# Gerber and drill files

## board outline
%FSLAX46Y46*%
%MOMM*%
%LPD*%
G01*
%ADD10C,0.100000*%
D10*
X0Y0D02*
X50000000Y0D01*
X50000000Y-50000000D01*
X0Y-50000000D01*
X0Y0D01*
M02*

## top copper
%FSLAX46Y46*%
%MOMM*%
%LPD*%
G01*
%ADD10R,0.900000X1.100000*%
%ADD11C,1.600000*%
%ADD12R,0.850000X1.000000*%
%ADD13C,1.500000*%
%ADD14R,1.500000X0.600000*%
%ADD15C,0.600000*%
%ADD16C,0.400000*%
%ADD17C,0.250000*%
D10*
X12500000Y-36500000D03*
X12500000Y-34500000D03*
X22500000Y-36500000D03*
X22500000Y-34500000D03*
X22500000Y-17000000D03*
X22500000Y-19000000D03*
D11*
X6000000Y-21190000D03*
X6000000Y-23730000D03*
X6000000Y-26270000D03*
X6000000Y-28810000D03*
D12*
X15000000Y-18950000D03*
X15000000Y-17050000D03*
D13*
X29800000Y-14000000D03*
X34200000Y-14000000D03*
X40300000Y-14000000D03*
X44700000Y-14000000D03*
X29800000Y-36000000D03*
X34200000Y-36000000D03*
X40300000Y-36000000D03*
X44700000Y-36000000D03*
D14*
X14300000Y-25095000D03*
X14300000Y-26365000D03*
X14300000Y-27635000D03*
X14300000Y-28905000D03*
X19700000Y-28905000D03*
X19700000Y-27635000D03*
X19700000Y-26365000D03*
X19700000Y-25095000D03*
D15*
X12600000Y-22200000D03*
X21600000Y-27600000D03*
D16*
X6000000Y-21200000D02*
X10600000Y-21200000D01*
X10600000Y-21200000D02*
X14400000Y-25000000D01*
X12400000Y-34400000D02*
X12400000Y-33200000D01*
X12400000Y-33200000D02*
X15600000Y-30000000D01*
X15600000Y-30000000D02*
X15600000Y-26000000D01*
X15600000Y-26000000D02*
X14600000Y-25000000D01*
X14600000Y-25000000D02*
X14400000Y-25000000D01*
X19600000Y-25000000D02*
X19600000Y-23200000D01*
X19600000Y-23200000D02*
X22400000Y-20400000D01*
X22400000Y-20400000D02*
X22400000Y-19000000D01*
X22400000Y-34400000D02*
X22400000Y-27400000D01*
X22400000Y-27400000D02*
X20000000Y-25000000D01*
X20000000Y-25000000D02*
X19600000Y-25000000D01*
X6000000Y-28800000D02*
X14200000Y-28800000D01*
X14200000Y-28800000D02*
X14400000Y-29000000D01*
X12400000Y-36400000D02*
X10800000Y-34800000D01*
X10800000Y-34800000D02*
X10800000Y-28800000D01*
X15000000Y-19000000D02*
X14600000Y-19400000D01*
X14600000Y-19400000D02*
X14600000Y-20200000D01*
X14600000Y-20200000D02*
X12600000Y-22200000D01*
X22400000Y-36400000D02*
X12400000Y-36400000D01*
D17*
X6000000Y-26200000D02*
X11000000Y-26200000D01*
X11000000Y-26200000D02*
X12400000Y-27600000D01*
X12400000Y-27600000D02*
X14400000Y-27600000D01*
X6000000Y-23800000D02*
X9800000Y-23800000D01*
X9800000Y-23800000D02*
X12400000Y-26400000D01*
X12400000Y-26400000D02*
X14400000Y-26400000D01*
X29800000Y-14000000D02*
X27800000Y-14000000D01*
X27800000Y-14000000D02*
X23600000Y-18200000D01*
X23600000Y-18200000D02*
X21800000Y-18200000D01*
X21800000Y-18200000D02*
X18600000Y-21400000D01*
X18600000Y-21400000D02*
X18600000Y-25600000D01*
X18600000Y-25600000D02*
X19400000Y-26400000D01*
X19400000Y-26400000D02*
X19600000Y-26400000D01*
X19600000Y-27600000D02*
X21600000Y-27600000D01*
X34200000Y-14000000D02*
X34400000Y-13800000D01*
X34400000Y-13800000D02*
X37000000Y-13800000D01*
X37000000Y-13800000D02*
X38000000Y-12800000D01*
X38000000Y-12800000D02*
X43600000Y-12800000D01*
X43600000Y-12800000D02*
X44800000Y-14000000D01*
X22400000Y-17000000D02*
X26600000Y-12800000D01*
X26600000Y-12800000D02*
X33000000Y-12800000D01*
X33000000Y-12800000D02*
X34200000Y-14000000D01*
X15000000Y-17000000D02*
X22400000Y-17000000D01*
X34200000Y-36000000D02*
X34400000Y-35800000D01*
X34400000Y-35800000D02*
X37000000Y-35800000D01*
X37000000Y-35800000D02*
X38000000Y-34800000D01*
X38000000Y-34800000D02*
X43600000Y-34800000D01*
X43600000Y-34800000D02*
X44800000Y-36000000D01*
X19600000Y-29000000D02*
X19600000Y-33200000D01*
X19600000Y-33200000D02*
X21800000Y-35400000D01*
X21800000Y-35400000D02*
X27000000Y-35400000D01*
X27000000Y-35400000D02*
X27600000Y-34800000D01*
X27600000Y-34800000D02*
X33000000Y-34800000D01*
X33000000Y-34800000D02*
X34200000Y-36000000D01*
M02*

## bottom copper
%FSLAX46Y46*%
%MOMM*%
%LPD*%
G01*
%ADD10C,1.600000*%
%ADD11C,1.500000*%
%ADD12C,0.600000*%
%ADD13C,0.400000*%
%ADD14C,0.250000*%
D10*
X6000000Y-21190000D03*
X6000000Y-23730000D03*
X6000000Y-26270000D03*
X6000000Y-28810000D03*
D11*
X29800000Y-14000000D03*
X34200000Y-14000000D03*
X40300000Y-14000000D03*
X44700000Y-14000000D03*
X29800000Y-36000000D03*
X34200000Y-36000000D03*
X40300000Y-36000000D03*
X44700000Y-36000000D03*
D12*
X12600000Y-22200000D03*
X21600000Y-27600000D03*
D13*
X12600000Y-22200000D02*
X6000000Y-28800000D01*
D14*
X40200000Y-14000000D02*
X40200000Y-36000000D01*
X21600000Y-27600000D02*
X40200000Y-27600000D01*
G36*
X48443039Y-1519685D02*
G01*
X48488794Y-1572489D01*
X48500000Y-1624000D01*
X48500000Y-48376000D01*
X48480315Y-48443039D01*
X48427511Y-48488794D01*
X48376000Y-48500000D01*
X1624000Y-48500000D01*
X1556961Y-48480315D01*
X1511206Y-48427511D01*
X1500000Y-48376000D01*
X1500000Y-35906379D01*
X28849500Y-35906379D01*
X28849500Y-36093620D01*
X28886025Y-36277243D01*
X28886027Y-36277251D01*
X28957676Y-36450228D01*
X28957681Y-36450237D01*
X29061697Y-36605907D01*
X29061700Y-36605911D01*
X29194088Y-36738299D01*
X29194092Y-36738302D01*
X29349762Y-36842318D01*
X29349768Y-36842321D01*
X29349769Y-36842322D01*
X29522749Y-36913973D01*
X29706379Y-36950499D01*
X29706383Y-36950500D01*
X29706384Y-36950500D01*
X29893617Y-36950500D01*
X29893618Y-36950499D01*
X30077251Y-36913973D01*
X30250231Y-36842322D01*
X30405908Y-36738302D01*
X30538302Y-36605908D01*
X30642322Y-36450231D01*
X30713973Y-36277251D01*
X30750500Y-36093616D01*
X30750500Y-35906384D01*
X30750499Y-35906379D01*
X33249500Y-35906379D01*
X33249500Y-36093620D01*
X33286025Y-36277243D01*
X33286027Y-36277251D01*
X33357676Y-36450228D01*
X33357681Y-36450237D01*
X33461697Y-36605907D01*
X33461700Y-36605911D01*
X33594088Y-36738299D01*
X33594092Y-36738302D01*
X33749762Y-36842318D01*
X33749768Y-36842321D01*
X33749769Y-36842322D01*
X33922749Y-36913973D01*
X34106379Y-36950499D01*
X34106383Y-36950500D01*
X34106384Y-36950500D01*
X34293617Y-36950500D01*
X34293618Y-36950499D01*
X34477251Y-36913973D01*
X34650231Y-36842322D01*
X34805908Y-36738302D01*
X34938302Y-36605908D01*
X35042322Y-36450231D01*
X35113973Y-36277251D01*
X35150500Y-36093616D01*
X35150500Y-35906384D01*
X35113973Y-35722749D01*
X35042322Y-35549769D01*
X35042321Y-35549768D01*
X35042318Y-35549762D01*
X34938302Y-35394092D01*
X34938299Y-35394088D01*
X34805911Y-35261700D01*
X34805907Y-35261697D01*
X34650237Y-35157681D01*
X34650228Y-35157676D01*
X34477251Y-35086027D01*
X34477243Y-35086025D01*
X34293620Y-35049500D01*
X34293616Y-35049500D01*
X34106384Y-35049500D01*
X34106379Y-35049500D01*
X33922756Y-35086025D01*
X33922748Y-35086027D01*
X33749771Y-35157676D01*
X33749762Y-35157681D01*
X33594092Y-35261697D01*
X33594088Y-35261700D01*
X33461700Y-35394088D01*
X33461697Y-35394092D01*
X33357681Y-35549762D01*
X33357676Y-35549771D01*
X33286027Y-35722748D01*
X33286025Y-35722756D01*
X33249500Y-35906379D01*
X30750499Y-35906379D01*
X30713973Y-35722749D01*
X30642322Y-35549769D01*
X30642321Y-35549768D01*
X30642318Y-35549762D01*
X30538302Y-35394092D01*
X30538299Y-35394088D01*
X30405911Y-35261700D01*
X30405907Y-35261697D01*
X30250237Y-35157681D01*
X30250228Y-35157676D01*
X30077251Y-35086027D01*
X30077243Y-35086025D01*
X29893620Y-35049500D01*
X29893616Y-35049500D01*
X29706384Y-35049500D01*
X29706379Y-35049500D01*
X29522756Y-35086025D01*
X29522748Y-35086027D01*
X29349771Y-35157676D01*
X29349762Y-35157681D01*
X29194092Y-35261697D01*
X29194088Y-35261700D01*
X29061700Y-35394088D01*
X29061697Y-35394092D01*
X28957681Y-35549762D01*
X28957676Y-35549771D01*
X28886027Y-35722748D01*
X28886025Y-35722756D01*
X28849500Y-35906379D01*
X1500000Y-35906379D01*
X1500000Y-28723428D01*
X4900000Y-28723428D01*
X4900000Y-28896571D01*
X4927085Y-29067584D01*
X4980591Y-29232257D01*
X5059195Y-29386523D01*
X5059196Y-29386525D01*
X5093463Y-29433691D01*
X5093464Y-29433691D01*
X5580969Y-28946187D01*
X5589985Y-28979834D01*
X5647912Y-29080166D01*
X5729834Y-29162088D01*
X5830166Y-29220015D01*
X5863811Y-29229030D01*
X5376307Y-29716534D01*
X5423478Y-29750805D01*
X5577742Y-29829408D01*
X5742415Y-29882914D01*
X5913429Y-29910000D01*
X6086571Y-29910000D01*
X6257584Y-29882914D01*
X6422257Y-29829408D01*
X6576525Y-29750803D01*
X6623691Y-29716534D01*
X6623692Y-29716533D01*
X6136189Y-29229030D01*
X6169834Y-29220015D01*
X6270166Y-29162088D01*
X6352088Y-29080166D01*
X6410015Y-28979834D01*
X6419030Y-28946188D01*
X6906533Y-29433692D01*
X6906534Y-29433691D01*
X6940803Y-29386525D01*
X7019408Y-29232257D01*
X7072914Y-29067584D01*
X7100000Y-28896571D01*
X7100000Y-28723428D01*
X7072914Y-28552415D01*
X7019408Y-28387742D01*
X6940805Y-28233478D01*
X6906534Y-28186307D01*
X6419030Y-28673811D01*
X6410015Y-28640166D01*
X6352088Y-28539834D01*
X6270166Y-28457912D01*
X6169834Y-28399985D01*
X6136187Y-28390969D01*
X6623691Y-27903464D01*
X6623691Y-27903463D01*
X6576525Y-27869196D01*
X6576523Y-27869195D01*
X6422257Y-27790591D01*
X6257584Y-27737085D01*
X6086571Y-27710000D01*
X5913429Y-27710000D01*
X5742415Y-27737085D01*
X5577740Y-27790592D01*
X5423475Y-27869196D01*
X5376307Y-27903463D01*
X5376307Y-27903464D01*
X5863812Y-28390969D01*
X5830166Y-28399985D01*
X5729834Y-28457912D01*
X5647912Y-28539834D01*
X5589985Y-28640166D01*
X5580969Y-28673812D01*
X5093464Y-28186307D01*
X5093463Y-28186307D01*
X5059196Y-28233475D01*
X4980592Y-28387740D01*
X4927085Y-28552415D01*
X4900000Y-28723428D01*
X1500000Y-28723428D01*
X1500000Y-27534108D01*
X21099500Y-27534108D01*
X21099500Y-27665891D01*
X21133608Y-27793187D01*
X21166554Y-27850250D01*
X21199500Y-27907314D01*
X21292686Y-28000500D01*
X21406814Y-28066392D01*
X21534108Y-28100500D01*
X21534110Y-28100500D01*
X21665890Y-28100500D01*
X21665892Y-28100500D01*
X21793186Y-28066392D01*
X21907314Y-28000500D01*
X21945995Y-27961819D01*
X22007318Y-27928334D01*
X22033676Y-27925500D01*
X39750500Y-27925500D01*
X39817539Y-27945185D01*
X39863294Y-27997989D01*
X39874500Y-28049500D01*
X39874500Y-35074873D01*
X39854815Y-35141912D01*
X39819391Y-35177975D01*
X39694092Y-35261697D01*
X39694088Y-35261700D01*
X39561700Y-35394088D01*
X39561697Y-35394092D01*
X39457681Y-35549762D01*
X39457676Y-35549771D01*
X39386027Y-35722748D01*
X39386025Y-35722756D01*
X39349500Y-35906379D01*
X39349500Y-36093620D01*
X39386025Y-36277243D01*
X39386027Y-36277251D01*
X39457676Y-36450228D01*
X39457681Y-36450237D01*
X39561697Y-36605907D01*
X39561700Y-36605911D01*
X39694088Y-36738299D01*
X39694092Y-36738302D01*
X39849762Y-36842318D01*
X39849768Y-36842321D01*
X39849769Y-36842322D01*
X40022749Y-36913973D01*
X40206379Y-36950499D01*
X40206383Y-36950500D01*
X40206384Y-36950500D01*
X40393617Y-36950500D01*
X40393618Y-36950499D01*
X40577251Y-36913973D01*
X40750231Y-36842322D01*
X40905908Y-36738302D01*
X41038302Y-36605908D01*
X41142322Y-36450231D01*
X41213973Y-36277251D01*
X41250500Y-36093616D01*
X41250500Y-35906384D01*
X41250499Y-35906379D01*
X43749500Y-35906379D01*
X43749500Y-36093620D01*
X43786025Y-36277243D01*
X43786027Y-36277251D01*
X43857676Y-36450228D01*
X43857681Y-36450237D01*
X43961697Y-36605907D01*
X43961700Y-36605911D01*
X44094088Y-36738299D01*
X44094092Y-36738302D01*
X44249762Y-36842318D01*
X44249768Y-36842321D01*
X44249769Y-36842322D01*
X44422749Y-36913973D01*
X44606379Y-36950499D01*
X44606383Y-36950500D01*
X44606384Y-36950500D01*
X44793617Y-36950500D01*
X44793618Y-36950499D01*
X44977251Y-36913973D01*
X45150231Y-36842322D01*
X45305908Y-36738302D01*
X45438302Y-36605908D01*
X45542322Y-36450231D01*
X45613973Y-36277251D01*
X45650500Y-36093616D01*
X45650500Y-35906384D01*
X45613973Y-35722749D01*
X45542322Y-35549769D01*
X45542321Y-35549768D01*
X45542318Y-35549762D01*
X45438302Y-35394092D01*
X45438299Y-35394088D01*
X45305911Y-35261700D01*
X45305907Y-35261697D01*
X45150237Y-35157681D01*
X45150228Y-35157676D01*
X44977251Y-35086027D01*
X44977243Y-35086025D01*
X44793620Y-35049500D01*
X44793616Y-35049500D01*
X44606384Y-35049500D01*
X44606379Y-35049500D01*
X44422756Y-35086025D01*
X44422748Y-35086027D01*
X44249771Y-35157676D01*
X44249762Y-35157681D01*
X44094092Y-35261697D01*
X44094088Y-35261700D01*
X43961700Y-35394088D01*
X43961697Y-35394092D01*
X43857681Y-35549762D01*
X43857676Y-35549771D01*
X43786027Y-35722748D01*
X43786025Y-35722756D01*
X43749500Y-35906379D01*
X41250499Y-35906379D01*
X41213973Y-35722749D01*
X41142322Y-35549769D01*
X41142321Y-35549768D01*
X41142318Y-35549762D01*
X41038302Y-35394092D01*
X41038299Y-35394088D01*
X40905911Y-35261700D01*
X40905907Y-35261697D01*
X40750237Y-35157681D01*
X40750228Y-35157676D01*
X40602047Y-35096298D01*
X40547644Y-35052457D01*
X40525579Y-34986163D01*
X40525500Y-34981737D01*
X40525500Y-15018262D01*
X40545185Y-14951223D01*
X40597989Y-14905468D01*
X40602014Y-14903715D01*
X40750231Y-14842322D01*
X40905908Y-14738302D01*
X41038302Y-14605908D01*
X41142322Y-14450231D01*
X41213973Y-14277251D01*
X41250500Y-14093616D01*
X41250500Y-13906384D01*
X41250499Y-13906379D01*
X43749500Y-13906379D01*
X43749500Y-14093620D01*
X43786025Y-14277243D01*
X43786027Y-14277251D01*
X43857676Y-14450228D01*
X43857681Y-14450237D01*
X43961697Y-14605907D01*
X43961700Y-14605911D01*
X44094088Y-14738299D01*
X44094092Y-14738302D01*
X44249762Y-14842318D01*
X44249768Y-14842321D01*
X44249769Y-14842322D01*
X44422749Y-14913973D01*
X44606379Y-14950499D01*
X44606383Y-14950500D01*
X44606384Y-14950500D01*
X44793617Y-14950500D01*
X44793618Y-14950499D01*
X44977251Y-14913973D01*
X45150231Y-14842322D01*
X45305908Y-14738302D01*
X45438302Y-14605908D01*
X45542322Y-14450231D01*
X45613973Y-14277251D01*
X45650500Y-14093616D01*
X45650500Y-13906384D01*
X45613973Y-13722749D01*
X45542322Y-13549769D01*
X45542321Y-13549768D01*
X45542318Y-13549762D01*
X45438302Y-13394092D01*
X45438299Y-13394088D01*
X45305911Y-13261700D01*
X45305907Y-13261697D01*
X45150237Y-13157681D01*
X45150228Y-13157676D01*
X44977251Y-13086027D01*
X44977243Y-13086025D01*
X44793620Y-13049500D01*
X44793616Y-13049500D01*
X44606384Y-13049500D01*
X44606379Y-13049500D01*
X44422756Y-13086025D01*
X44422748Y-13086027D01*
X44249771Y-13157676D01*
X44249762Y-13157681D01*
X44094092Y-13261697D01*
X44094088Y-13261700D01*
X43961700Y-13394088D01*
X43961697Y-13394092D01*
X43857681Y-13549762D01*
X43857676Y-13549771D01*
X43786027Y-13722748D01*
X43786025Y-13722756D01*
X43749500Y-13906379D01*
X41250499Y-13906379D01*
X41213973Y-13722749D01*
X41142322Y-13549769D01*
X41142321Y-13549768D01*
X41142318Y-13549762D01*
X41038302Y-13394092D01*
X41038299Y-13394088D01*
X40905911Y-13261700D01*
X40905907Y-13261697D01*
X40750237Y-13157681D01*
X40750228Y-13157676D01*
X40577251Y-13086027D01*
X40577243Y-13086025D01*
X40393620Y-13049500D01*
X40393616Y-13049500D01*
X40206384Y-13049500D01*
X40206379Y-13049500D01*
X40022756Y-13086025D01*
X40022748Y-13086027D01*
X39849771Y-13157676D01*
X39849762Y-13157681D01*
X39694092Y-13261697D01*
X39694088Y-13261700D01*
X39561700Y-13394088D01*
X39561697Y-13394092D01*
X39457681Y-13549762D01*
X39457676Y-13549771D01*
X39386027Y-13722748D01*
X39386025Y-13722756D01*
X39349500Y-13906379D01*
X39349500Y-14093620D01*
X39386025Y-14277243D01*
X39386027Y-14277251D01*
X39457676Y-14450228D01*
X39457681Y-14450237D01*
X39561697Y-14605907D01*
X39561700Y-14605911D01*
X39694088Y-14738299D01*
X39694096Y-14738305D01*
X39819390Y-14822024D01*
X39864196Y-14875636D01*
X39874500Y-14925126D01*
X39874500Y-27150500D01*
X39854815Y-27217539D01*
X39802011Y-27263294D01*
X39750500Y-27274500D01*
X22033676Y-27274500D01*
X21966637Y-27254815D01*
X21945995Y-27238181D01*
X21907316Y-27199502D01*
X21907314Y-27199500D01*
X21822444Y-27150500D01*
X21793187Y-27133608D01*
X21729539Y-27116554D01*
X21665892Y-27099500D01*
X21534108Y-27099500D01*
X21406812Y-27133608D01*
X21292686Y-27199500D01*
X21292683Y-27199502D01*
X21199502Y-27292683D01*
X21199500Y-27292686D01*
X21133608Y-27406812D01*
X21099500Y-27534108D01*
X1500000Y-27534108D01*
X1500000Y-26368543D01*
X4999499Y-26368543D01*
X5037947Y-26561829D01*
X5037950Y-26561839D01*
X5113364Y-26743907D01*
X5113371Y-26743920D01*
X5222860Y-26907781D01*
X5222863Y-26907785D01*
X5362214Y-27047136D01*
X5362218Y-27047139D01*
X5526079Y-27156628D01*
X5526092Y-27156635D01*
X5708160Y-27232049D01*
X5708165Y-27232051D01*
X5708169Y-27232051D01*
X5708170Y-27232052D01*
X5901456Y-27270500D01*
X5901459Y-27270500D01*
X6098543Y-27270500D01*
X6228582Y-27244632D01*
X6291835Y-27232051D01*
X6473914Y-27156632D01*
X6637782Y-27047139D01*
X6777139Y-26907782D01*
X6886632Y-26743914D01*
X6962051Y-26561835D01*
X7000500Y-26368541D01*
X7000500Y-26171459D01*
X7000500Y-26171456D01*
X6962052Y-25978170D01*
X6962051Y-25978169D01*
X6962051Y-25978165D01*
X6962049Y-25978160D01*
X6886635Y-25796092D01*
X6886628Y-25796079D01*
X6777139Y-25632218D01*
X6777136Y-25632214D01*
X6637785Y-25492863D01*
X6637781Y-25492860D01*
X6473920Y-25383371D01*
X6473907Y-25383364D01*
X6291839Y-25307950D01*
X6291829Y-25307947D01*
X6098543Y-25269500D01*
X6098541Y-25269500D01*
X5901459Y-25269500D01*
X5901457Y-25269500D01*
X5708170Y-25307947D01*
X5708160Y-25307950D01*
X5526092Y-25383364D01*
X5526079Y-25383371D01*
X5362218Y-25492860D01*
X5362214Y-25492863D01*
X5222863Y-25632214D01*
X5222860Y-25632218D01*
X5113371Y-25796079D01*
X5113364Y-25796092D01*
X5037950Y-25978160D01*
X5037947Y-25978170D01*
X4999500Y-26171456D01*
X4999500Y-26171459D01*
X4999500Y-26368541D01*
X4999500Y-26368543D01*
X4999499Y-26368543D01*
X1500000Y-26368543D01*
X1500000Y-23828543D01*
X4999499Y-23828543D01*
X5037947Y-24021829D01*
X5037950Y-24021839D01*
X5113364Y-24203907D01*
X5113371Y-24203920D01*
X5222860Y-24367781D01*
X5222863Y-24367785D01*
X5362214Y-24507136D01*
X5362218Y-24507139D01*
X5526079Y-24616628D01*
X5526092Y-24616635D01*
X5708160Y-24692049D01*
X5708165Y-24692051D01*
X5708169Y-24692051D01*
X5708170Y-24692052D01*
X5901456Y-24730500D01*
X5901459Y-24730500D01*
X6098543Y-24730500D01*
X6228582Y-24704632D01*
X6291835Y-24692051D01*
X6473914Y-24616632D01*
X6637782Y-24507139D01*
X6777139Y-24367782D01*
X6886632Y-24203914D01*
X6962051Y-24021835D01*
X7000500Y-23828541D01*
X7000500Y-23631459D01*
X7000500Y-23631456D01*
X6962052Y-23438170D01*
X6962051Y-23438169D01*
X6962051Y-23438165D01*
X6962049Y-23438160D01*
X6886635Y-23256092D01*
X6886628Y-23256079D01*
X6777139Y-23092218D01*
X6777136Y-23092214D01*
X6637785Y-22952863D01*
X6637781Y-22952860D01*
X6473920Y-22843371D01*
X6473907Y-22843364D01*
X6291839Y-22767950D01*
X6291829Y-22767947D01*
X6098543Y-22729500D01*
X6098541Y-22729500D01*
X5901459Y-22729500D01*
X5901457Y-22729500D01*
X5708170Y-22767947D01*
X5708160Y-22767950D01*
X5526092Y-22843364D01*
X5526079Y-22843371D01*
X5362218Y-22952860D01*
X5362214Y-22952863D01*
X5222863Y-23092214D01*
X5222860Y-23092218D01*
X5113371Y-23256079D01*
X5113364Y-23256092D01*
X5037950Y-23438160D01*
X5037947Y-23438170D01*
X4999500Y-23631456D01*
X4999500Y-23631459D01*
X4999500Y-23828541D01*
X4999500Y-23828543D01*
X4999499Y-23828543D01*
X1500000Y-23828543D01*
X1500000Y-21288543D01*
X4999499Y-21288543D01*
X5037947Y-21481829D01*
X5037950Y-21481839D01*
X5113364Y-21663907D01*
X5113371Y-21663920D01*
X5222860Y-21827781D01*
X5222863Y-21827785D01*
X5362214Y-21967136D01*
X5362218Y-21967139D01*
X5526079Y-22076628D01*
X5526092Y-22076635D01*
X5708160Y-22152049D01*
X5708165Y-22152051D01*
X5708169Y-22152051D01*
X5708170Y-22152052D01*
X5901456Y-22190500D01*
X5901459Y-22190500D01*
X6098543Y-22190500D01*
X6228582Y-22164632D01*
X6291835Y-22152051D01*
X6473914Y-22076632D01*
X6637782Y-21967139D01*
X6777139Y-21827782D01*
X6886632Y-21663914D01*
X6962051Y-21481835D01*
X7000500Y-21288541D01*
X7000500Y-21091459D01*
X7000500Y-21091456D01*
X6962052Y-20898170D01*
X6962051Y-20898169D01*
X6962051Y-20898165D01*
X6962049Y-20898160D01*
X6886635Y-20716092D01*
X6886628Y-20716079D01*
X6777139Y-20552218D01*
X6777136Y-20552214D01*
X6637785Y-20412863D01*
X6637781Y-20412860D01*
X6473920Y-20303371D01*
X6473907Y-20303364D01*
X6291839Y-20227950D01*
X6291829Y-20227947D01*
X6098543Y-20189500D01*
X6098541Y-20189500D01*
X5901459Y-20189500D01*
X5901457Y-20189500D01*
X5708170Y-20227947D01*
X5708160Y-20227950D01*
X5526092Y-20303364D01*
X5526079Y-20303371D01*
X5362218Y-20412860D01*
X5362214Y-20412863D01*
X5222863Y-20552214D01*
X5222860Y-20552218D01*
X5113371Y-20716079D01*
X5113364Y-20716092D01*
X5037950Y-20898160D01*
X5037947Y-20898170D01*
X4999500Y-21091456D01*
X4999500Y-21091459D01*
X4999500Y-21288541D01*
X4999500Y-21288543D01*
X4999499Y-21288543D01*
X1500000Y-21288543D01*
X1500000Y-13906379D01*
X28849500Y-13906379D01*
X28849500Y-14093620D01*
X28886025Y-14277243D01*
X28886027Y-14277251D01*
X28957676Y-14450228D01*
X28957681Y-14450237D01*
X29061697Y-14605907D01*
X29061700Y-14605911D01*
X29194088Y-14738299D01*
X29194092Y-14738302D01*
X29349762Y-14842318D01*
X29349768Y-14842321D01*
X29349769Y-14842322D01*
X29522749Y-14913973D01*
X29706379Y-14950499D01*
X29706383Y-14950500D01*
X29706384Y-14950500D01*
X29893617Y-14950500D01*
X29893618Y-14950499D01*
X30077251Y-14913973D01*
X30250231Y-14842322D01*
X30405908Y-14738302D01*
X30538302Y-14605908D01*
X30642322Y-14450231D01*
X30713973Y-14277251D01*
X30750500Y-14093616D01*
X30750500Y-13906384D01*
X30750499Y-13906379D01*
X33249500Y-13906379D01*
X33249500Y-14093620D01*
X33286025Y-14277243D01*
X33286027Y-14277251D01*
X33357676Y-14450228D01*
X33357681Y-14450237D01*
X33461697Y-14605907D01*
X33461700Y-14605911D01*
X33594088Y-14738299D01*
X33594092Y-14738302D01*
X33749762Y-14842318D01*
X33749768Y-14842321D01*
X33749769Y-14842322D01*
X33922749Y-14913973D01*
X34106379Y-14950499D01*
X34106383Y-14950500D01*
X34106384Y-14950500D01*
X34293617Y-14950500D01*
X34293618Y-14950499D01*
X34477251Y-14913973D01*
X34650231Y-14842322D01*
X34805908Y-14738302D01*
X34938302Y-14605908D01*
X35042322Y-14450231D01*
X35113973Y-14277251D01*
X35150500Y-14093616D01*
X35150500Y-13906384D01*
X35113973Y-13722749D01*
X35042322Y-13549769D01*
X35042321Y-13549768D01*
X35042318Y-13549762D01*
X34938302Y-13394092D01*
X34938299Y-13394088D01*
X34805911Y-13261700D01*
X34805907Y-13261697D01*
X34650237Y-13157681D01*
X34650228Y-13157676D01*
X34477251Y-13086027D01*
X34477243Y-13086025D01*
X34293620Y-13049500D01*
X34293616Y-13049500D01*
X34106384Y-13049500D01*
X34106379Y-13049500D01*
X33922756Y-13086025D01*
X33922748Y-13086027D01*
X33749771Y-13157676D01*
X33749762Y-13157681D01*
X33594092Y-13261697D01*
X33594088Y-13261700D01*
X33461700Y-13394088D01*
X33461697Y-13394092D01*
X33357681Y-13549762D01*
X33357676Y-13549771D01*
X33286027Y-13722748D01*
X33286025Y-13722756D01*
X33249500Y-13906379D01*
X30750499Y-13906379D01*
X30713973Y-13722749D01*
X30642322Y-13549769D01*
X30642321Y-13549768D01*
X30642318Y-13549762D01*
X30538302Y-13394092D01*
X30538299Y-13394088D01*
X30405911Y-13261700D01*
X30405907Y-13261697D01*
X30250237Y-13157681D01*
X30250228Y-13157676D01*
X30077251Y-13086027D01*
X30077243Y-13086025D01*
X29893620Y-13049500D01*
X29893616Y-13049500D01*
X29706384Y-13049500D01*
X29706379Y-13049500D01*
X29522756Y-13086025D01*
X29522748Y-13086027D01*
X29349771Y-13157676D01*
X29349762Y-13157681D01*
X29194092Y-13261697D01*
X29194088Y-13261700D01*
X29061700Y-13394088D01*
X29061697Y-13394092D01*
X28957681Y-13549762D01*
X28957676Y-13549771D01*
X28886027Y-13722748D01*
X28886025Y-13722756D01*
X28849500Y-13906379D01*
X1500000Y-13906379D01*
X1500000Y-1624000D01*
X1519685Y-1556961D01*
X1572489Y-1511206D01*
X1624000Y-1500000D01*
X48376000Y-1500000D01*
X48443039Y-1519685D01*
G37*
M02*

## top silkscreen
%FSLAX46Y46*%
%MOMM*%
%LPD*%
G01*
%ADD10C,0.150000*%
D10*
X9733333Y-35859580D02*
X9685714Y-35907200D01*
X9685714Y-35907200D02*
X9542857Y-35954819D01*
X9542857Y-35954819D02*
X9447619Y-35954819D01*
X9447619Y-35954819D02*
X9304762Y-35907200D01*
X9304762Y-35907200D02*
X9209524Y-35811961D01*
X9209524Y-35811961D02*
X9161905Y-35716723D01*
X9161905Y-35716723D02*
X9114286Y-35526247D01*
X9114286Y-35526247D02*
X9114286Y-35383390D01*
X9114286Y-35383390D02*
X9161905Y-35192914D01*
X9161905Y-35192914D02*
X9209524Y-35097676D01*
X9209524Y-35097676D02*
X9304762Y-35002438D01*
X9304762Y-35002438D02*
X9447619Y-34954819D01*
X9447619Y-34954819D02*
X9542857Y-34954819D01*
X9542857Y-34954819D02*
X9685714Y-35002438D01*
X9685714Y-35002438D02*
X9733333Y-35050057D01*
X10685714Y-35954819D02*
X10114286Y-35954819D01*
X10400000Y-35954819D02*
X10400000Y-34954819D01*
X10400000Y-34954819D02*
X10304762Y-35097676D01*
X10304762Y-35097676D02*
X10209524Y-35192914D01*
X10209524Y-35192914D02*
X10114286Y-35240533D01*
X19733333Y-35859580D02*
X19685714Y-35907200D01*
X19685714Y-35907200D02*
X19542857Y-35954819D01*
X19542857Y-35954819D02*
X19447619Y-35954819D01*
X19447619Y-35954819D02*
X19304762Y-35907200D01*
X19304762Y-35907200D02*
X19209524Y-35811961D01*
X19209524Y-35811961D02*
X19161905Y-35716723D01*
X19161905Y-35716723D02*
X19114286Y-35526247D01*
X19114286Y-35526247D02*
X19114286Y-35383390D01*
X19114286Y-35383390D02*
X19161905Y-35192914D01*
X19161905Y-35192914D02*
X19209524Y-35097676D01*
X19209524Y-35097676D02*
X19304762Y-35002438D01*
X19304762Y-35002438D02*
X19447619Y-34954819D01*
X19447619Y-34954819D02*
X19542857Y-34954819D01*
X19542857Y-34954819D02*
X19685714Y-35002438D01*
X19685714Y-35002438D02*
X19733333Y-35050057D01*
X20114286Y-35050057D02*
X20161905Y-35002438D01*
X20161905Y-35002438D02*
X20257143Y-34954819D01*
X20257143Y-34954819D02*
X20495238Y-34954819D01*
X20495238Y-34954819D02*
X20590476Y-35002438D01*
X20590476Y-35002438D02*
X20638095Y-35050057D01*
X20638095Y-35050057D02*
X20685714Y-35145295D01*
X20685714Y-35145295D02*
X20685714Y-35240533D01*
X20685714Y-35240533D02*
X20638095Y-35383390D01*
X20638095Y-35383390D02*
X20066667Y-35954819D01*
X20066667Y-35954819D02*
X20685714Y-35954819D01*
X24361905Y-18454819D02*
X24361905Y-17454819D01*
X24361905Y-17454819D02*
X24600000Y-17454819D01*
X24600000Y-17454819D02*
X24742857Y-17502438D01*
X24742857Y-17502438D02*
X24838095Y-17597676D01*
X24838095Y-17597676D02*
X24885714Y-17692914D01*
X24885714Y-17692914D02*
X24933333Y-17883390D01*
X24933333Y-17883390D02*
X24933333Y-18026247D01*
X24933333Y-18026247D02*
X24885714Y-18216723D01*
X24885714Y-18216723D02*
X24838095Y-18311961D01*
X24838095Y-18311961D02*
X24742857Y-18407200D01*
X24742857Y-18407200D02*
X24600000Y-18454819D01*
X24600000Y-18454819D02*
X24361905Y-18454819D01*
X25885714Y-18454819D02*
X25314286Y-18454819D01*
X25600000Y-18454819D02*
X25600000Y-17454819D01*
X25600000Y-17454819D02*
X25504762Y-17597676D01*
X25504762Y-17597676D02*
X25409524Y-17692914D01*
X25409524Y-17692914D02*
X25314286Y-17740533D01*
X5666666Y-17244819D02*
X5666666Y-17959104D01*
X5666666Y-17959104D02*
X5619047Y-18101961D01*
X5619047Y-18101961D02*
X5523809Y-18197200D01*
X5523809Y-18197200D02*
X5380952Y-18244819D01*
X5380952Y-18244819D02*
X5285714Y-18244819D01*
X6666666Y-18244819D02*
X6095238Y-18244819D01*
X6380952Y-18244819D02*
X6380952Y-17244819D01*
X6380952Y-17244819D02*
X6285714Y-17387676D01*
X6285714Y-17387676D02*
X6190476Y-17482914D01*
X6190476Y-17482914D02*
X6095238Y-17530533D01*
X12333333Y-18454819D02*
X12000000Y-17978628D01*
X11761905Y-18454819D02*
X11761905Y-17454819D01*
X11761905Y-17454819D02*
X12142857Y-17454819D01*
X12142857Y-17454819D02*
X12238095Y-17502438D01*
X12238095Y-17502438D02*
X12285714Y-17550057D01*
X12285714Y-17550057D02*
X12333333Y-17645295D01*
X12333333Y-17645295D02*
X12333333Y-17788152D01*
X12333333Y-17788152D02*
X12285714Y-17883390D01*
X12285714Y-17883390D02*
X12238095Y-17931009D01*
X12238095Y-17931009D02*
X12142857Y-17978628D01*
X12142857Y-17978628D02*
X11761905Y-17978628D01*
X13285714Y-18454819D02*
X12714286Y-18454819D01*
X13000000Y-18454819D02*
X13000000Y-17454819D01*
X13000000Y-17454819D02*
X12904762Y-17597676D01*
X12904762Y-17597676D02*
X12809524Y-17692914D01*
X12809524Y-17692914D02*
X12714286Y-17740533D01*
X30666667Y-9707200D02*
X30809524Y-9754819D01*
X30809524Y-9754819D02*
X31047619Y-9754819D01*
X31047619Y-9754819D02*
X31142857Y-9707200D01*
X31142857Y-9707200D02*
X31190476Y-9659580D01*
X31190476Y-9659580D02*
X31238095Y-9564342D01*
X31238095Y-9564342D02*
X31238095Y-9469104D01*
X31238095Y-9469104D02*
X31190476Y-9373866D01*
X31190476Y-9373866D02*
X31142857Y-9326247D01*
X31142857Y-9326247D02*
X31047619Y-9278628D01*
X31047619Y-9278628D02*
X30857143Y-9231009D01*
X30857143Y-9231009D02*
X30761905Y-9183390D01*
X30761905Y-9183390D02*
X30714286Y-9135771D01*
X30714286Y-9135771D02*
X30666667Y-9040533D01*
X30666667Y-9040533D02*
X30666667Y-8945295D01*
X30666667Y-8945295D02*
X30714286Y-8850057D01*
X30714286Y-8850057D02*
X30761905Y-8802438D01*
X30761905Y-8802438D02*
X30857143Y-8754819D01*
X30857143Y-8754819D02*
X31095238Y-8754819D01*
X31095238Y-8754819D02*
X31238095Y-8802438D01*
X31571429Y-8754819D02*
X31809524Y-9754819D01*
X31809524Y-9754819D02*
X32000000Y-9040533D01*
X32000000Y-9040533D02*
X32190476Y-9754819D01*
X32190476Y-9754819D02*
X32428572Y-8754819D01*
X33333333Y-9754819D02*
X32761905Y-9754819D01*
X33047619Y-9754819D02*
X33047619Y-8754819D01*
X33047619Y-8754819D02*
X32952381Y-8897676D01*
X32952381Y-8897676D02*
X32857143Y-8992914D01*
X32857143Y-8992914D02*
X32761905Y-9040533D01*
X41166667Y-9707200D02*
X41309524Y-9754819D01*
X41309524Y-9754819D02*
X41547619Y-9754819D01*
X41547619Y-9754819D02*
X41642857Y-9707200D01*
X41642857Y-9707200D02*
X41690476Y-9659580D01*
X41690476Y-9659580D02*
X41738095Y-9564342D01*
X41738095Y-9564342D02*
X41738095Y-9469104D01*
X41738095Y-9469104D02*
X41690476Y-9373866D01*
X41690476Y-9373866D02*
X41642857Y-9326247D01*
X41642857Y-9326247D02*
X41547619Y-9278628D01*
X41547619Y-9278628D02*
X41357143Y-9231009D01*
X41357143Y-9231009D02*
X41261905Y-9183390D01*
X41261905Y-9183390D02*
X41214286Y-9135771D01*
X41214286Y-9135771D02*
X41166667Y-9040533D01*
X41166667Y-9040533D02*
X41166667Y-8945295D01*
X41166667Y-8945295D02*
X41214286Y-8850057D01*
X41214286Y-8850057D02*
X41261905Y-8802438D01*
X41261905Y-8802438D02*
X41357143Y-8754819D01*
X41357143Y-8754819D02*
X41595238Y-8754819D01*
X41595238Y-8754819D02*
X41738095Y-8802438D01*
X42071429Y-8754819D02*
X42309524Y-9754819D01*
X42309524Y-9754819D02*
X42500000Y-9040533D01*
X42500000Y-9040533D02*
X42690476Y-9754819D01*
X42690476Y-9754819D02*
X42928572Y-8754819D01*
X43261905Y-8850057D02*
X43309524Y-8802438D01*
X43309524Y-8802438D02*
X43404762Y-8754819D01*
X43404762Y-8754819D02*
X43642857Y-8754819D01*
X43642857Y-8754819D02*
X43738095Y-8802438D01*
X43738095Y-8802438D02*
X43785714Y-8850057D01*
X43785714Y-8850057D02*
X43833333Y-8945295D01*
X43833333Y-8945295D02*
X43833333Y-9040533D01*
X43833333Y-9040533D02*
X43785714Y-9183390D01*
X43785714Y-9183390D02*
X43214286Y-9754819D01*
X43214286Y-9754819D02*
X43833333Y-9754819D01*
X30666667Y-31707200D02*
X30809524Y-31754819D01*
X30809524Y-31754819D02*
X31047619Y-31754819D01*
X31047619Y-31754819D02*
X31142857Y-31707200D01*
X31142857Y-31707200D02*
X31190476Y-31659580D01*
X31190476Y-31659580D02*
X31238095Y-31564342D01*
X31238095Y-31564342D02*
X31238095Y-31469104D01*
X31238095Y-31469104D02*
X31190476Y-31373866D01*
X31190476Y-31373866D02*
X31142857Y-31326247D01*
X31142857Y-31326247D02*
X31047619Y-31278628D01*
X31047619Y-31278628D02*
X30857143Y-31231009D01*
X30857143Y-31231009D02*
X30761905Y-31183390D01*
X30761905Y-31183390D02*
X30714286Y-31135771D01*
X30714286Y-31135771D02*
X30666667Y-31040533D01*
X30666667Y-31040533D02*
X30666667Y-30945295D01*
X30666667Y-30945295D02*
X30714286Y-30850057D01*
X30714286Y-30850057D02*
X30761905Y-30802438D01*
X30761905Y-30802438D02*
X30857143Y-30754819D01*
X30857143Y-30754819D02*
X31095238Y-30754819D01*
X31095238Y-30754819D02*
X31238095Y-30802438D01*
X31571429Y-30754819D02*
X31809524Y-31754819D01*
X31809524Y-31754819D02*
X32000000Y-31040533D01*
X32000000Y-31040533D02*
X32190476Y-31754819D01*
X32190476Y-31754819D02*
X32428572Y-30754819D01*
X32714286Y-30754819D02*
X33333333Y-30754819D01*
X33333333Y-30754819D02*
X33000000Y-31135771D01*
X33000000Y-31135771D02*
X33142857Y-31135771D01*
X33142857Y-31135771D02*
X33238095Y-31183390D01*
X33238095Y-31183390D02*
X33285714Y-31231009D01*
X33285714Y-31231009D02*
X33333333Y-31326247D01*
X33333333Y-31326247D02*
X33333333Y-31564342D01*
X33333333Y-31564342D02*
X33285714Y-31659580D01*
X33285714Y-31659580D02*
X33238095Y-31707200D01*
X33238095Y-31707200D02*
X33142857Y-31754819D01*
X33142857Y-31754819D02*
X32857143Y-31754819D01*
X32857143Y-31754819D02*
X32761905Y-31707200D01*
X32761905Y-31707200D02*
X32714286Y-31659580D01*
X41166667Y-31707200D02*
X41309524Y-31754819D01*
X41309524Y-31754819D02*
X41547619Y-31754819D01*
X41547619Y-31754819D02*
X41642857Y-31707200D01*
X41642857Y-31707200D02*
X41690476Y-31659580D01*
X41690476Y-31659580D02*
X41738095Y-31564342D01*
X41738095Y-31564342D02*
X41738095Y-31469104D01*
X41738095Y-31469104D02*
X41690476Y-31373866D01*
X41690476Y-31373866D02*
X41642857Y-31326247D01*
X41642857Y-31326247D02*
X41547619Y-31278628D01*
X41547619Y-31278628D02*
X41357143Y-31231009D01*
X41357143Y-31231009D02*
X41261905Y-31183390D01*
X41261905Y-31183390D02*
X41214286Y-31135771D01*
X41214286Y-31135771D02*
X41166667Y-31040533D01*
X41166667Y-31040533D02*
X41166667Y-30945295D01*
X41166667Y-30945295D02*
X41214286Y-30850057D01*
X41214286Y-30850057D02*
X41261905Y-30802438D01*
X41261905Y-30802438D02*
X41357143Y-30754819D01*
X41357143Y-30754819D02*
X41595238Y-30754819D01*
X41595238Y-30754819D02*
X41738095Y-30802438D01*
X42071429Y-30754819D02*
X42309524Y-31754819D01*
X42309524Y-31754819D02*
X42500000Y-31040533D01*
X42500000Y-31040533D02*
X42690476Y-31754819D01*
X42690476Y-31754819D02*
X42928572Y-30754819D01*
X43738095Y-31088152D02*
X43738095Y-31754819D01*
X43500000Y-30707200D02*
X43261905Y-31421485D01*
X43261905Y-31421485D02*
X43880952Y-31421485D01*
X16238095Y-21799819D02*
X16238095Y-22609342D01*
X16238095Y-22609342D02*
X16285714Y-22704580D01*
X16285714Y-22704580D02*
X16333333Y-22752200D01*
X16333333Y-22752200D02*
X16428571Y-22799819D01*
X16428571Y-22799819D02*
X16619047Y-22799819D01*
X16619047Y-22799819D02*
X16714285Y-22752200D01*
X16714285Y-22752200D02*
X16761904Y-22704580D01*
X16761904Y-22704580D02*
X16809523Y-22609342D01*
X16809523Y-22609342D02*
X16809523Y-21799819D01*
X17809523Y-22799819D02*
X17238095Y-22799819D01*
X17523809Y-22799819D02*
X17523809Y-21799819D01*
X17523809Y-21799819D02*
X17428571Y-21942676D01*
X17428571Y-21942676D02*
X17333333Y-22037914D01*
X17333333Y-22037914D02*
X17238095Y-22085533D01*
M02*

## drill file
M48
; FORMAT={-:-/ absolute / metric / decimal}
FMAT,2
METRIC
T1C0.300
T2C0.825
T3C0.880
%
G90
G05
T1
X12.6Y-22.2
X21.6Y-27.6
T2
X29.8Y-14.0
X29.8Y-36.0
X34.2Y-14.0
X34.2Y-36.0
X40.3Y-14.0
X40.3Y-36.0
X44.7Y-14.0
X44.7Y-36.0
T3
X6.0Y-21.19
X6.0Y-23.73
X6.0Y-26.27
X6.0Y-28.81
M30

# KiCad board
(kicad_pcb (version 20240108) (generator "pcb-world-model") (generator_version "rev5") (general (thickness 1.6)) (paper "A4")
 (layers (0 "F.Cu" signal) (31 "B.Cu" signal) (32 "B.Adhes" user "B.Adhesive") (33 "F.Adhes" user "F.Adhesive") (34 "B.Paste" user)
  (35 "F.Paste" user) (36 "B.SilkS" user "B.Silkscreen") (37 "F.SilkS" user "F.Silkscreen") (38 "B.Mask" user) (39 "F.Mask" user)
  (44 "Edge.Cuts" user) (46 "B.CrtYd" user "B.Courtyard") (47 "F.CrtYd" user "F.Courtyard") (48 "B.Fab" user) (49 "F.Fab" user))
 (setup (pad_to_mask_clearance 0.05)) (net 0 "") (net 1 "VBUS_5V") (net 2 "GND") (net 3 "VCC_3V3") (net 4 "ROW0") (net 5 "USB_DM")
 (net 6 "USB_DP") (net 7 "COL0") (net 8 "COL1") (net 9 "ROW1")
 (gr_rect (start 0.0 0.0) (end 50.0000 50.0000) (stroke (width 0.1) (type default)) (fill none) (layer "Edge.Cuts"))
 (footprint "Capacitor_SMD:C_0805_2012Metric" (layer "F.Cu") (at 12.5000 35.5000 90)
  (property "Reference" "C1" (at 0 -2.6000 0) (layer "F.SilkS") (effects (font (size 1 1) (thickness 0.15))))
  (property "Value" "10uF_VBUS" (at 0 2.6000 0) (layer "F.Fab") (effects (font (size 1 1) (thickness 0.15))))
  (pad "1" smd rect (at -1.0000 0.0000) (size 0.9000 1.1000) (layers "F.Cu" "F.Paste" "F.Mask") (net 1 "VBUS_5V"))
  (pad "2" smd rect (at 1.0000 0.0000) (size 0.9000 1.1000) (layers "F.Cu" "F.Paste" "F.Mask") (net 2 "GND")))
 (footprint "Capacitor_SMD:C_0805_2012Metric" (layer "F.Cu") (at 22.5000 35.5000 90)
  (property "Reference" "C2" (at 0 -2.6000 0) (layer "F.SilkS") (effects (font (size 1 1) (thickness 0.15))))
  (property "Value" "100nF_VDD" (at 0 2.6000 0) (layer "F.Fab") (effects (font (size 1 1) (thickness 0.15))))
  (pad "1" smd rect (at -1.0000 0.0000) (size 0.9000 1.1000) (layers "F.Cu" "F.Paste" "F.Mask") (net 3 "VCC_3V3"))
  (pad "2" smd rect (at 1.0000 0.0000) (size 0.9000 1.1000) (layers "F.Cu" "F.Paste" "F.Mask") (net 2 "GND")))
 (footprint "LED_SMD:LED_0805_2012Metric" (layer "F.Cu") (at 22.5000 18.0000 270)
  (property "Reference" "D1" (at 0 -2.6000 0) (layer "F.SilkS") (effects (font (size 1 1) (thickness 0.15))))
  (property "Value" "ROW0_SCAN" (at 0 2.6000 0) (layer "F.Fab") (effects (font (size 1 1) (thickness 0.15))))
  (pad "1" smd rect (at -1.0000 0.0000) (size 0.9000 1.1000) (layers "F.Cu" "F.Paste" "F.Mask") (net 3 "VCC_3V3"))
  (pad "2" smd rect (at 1.0000 0.0000) (size 0.9000 1.1000) (layers "F.Cu" "F.Paste" "F.Mask") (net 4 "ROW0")))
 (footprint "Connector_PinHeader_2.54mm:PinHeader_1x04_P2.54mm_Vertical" (layer "F.Cu") (at 6.0000 25.0000 0) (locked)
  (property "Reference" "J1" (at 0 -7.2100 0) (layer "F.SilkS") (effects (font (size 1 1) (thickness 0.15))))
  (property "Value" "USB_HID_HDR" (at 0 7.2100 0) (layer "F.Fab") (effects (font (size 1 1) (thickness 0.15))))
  (pad "1" thru_hole circle (at 0.0000 -3.8100) (size 1.6000 1.6000) (drill 0.8800) (layers "*.Cu" "*.Mask") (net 1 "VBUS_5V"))
  (pad "2" thru_hole circle (at 0.0000 -1.2700) (size 1.6000 1.6000) (drill 0.8800) (layers "*.Cu" "*.Mask") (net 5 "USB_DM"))
  (pad "3" thru_hole circle (at 0.0000 1.2700) (size 1.6000 1.6000) (drill 0.8800) (layers "*.Cu" "*.Mask") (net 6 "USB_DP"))
  (pad "4" thru_hole circle (at 0.0000 3.8100) (size 1.6000 1.6000) (drill 0.8800) (layers "*.Cu" "*.Mask") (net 2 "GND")))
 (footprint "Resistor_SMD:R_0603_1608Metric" (layer "F.Cu") (at 15.0000 18.0000 90)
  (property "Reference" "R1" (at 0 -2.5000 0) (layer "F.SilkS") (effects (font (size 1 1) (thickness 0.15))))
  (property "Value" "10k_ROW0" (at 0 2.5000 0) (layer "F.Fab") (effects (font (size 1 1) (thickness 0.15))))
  (pad "1" smd rect (at -0.9500 0.0000) (size 0.8500 1.0000) (layers "F.Cu" "F.Paste" "F.Mask") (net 4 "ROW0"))
  (pad "2" smd rect (at 0.9500 0.0000) (size 0.8500 1.0000) (layers "F.Cu" "F.Paste" "F.Mask") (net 2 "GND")))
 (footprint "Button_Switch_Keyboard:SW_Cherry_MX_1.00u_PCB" (layer "F.Cu") (at 32.0000 14.0000 0) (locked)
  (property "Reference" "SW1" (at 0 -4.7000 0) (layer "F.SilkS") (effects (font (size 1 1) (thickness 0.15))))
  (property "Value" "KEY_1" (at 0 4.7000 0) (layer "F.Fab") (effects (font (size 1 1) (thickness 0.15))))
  (pad "1" thru_hole circle (at -2.2000 0.0000) (size 1.5000 1.5000) (drill 0.8250) (layers "*.Cu" "*.Mask") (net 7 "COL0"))
  (pad "2" thru_hole circle (at 2.2000 0.0000) (size 1.5000 1.5000) (drill 0.8250) (layers "*.Cu" "*.Mask") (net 4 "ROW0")))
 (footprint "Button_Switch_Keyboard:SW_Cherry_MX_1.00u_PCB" (layer "F.Cu") (at 42.5000 14.0000 0) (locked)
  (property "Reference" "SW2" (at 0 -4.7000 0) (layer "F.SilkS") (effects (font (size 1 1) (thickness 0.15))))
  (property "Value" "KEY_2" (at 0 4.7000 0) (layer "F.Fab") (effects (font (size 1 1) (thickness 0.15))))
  (pad "1" thru_hole circle (at -2.2000 0.0000) (size 1.5000 1.5000) (drill 0.8250) (layers "*.Cu" "*.Mask") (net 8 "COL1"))
  (pad "2" thru_hole circle (at 2.2000 0.0000) (size 1.5000 1.5000) (drill 0.8250) (layers "*.Cu" "*.Mask") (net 4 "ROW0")))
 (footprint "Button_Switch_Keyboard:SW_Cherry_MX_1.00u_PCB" (layer "F.Cu") (at 32.0000 36.0000 0) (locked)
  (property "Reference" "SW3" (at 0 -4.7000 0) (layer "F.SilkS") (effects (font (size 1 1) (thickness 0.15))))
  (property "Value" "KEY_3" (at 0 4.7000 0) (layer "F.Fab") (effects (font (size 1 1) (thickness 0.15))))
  (pad "1" thru_hole circle (at -2.2000 0.0000) (size 1.5000 1.5000) (drill 0.8250) (layers "*.Cu" "*.Mask") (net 7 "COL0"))
  (pad "2" thru_hole circle (at 2.2000 0.0000) (size 1.5000 1.5000) (drill 0.8250) (layers "*.Cu" "*.Mask") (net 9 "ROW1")))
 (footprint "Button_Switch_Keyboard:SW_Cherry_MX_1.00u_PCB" (layer "F.Cu") (at 42.5000 36.0000 0) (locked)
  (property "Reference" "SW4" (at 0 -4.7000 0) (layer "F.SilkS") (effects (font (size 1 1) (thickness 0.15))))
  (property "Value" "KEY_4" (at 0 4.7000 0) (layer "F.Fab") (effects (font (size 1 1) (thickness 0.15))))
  (pad "1" thru_hole circle (at -2.2000 0.0000) (size 1.5000 1.5000) (drill 0.8250) (layers "*.Cu" "*.Mask") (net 8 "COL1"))
  (pad "2" thru_hole circle (at 2.2000 0.0000) (size 1.5000 1.5000) (drill 0.8250) (layers "*.Cu" "*.Mask") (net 9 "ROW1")))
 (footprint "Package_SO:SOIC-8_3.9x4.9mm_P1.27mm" (layer "F.Cu") (at 17.0000 27.0000 0)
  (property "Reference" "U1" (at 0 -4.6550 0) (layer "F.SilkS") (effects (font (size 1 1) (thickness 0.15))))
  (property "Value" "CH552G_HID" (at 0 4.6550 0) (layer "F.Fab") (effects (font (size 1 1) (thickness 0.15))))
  (pad "1" smd rect (at -2.7000 -1.9050) (size 1.5000 0.6000) (layers "F.Cu" "F.Paste" "F.Mask") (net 1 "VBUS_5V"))
  (pad "2" smd rect (at -2.7000 -0.6350) (size 1.5000 0.6000) (layers "F.Cu" "F.Paste" "F.Mask") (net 5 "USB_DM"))
  (pad "3" smd rect (at -2.7000 0.6350) (size 1.5000 0.6000) (layers "F.Cu" "F.Paste" "F.Mask") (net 6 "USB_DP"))
  (pad "4" smd rect (at -2.7000 1.9050) (size 1.5000 0.6000) (layers "F.Cu" "F.Paste" "F.Mask") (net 2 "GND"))
  (pad "5" smd rect (at 2.7000 1.9050) (size 1.5000 0.6000) (layers "F.Cu" "F.Paste" "F.Mask") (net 9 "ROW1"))
  (pad "6" smd rect (at 2.7000 0.6350) (size 1.5000 0.6000) (layers "F.Cu" "F.Paste" "F.Mask") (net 8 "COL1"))
  (pad "7" smd rect (at 2.7000 -0.6350) (size 1.5000 0.6000) (layers "F.Cu" "F.Paste" "F.Mask") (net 7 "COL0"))
  (pad "8" smd rect (at 2.7000 -1.9050) (size 1.5000 0.6000) (layers "F.Cu" "F.Paste" "F.Mask") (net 3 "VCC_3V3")))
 (segment (start 6.0000 21.2000) (end 10.6000 21.2000) (width 0.4000) (layer "F.Cu") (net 1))
 (segment (start 10.6000 21.2000) (end 14.4000 25.0000) (width 0.4000) (layer "F.Cu") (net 1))
 (segment (start 12.4000 34.4000) (end 12.4000 33.2000) (width 0.4000) (layer "F.Cu") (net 1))
 (segment (start 12.4000 33.2000) (end 15.6000 30.0000) (width 0.4000) (layer "F.Cu") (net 1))
 (segment (start 15.6000 30.0000) (end 15.6000 26.0000) (width 0.4000) (layer "F.Cu") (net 1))
 (segment (start 15.6000 26.0000) (end 14.6000 25.0000) (width 0.4000) (layer "F.Cu") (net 1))
 (segment (start 14.6000 25.0000) (end 14.4000 25.0000) (width 0.4000) (layer "F.Cu") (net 1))
 (segment (start 19.6000 25.0000) (end 19.6000 23.2000) (width 0.4000) (layer "F.Cu") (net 3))
 (segment (start 19.6000 23.2000) (end 22.4000 20.4000) (width 0.4000) (layer "F.Cu") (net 3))
 (segment (start 22.4000 20.4000) (end 22.4000 19.0000) (width 0.4000) (layer "F.Cu") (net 3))
 (segment (start 22.4000 34.4000) (end 22.4000 27.4000) (width 0.4000) (layer "F.Cu") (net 3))
 (segment (start 22.4000 27.4000) (end 20.0000 25.0000) (width 0.4000) (layer "F.Cu") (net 3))
 (segment (start 20.0000 25.0000) (end 19.6000 25.0000) (width 0.4000) (layer "F.Cu") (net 3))
 (segment (start 6.0000 28.8000) (end 14.2000 28.8000) (width 0.4000) (layer "F.Cu") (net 2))
 (segment (start 14.2000 28.8000) (end 14.4000 29.0000) (width 0.4000) (layer "F.Cu") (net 2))
 (segment (start 12.4000 36.4000) (end 10.8000 34.8000) (width 0.4000) (layer "F.Cu") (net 2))
 (segment (start 10.8000 34.8000) (end 10.8000 28.8000) (width 0.4000) (layer "F.Cu") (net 2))
 (segment (start 15.0000 19.0000) (end 14.6000 19.4000) (width 0.4000) (layer "F.Cu") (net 2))
 (segment (start 14.6000 19.4000) (end 14.6000 20.2000) (width 0.4000) (layer "F.Cu") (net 2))
 (segment (start 14.6000 20.2000) (end 12.6000 22.2000) (width 0.4000) (layer "F.Cu") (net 2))
 (segment (start 12.6000 22.2000) (end 6.0000 28.8000) (width 0.4000) (layer "B.Cu") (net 2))
 (segment (start 22.4000 36.4000) (end 12.4000 36.4000) (width 0.4000) (layer "F.Cu") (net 2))
 (segment (start 6.0000 26.2000) (end 11.0000 26.2000) (width 0.2500) (layer "F.Cu") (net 6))
 (segment (start 11.0000 26.2000) (end 12.4000 27.6000) (width 0.2500) (layer "F.Cu") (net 6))
 (segment (start 12.4000 27.6000) (end 14.4000 27.6000) (width 0.2500) (layer "F.Cu") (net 6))
 (segment (start 6.0000 23.8000) (end 9.8000 23.8000) (width 0.2500) (layer "F.Cu") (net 5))
 (segment (start 9.8000 23.8000) (end 12.4000 26.4000) (width 0.2500) (layer "F.Cu") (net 5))
 (segment (start 12.4000 26.4000) (end 14.4000 26.4000) (width 0.2500) (layer "F.Cu") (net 5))
 (segment (start 29.8000 14.0000) (end 27.8000 14.0000) (width 0.2500) (layer "F.Cu") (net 7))
 (segment (start 27.8000 14.0000) (end 23.6000 18.2000) (width 0.2500) (layer "F.Cu") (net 7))
 (segment (start 23.6000 18.2000) (end 21.8000 18.2000) (width 0.2500) (layer "F.Cu") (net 7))
 (segment (start 21.8000 18.2000) (end 18.6000 21.4000) (width 0.2500) (layer "F.Cu") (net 7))
 (segment (start 18.6000 21.4000) (end 18.6000 25.6000) (width 0.2500) (layer "F.Cu") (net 7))
 (segment (start 18.6000 25.6000) (end 19.4000 26.4000) (width 0.2500) (layer "F.Cu") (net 7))
 (segment (start 19.4000 26.4000) (end 19.6000 26.4000) (width 0.2500) (layer "F.Cu") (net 7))
 (segment (start 40.2000 14.0000) (end 40.2000 36.0000) (width 0.2500) (layer "B.Cu") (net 8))
 (segment (start 19.6000 27.6000) (end 21.6000 27.6000) (width 0.2500) (layer "F.Cu") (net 8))
 (segment (start 21.6000 27.6000) (end 40.2000 27.6000) (width 0.2500) (layer "B.Cu") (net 8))
 (segment (start 34.2000 14.0000) (end 34.4000 13.8000) (width 0.2500) (layer "F.Cu") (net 4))
 (segment (start 34.4000 13.8000) (end 37.0000 13.8000) (width 0.2500) (layer "F.Cu") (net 4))
 (segment (start 37.0000 13.8000) (end 38.0000 12.8000) (width 0.2500) (layer "F.Cu") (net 4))
 (segment (start 38.0000 12.8000) (end 43.6000 12.8000) (width 0.2500) (layer "F.Cu") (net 4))
 (segment (start 43.6000 12.8000) (end 44.8000 14.0000) (width 0.2500) (layer "F.Cu") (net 4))
 (segment (start 22.4000 17.0000) (end 26.6000 12.8000) (width 0.2500) (layer "F.Cu") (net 4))
 (segment (start 26.6000 12.8000) (end 33.0000 12.8000) (width 0.2500) (layer "F.Cu") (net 4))
 (segment (start 33.0000 12.8000) (end 34.2000 14.0000) (width 0.2500) (layer "F.Cu") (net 4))
 (segment (start 15.0000 17.0000) (end 22.4000 17.0000) (width 0.2500) (layer "F.Cu") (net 4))
 (segment (start 34.2000 36.0000) (end 34.4000 35.8000) (width 0.2500) (layer "F.Cu") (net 9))
 (segment (start 34.4000 35.8000) (end 37.0000 35.8000) (width 0.2500) (layer "F.Cu") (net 9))
 (segment (start 37.0000 35.8000) (end 38.0000 34.8000) (width 0.2500) (layer "F.Cu") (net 9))
 (segment (start 38.0000 34.8000) (end 43.6000 34.8000) (width 0.2500) (layer "F.Cu") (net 9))
 (segment (start 43.6000 34.8000) (end 44.8000 36.0000) (width 0.2500) (layer "F.Cu") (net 9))
 (segment (start 19.6000 29.0000) (end 19.6000 33.2000) (width 0.2500) (layer "F.Cu") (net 9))
 (segment (start 19.6000 33.2000) (end 21.8000 35.4000) (width 0.2500) (layer "F.Cu") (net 9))
 (segment (start 21.8000 35.4000) (end 27.0000 35.4000) (width 0.2500) (layer "F.Cu") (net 9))
 (segment (start 27.0000 35.4000) (end 27.6000 34.8000) (width 0.2500) (layer "F.Cu") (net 9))
 (segment (start 27.6000 34.8000) (end 33.0000 34.8000) (width 0.2500) (layer "F.Cu") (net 9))
 (segment (start 33.0000 34.8000) (end 34.2000 36.0000) (width 0.2500) (layer "F.Cu") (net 9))
 (via (at 12.6000 22.2000) (size 0.6000) (drill 0.3000) (layers "F.Cu" "B.Cu") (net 2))
 (via (at 21.6000 27.6000) (size 0.6000) (drill 0.3000) (layers "F.Cu" "B.Cu") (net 8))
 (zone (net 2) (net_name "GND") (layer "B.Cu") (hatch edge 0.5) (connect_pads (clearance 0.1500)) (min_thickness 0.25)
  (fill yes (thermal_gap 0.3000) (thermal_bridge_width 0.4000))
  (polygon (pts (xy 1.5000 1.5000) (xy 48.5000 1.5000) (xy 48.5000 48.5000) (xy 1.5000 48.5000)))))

